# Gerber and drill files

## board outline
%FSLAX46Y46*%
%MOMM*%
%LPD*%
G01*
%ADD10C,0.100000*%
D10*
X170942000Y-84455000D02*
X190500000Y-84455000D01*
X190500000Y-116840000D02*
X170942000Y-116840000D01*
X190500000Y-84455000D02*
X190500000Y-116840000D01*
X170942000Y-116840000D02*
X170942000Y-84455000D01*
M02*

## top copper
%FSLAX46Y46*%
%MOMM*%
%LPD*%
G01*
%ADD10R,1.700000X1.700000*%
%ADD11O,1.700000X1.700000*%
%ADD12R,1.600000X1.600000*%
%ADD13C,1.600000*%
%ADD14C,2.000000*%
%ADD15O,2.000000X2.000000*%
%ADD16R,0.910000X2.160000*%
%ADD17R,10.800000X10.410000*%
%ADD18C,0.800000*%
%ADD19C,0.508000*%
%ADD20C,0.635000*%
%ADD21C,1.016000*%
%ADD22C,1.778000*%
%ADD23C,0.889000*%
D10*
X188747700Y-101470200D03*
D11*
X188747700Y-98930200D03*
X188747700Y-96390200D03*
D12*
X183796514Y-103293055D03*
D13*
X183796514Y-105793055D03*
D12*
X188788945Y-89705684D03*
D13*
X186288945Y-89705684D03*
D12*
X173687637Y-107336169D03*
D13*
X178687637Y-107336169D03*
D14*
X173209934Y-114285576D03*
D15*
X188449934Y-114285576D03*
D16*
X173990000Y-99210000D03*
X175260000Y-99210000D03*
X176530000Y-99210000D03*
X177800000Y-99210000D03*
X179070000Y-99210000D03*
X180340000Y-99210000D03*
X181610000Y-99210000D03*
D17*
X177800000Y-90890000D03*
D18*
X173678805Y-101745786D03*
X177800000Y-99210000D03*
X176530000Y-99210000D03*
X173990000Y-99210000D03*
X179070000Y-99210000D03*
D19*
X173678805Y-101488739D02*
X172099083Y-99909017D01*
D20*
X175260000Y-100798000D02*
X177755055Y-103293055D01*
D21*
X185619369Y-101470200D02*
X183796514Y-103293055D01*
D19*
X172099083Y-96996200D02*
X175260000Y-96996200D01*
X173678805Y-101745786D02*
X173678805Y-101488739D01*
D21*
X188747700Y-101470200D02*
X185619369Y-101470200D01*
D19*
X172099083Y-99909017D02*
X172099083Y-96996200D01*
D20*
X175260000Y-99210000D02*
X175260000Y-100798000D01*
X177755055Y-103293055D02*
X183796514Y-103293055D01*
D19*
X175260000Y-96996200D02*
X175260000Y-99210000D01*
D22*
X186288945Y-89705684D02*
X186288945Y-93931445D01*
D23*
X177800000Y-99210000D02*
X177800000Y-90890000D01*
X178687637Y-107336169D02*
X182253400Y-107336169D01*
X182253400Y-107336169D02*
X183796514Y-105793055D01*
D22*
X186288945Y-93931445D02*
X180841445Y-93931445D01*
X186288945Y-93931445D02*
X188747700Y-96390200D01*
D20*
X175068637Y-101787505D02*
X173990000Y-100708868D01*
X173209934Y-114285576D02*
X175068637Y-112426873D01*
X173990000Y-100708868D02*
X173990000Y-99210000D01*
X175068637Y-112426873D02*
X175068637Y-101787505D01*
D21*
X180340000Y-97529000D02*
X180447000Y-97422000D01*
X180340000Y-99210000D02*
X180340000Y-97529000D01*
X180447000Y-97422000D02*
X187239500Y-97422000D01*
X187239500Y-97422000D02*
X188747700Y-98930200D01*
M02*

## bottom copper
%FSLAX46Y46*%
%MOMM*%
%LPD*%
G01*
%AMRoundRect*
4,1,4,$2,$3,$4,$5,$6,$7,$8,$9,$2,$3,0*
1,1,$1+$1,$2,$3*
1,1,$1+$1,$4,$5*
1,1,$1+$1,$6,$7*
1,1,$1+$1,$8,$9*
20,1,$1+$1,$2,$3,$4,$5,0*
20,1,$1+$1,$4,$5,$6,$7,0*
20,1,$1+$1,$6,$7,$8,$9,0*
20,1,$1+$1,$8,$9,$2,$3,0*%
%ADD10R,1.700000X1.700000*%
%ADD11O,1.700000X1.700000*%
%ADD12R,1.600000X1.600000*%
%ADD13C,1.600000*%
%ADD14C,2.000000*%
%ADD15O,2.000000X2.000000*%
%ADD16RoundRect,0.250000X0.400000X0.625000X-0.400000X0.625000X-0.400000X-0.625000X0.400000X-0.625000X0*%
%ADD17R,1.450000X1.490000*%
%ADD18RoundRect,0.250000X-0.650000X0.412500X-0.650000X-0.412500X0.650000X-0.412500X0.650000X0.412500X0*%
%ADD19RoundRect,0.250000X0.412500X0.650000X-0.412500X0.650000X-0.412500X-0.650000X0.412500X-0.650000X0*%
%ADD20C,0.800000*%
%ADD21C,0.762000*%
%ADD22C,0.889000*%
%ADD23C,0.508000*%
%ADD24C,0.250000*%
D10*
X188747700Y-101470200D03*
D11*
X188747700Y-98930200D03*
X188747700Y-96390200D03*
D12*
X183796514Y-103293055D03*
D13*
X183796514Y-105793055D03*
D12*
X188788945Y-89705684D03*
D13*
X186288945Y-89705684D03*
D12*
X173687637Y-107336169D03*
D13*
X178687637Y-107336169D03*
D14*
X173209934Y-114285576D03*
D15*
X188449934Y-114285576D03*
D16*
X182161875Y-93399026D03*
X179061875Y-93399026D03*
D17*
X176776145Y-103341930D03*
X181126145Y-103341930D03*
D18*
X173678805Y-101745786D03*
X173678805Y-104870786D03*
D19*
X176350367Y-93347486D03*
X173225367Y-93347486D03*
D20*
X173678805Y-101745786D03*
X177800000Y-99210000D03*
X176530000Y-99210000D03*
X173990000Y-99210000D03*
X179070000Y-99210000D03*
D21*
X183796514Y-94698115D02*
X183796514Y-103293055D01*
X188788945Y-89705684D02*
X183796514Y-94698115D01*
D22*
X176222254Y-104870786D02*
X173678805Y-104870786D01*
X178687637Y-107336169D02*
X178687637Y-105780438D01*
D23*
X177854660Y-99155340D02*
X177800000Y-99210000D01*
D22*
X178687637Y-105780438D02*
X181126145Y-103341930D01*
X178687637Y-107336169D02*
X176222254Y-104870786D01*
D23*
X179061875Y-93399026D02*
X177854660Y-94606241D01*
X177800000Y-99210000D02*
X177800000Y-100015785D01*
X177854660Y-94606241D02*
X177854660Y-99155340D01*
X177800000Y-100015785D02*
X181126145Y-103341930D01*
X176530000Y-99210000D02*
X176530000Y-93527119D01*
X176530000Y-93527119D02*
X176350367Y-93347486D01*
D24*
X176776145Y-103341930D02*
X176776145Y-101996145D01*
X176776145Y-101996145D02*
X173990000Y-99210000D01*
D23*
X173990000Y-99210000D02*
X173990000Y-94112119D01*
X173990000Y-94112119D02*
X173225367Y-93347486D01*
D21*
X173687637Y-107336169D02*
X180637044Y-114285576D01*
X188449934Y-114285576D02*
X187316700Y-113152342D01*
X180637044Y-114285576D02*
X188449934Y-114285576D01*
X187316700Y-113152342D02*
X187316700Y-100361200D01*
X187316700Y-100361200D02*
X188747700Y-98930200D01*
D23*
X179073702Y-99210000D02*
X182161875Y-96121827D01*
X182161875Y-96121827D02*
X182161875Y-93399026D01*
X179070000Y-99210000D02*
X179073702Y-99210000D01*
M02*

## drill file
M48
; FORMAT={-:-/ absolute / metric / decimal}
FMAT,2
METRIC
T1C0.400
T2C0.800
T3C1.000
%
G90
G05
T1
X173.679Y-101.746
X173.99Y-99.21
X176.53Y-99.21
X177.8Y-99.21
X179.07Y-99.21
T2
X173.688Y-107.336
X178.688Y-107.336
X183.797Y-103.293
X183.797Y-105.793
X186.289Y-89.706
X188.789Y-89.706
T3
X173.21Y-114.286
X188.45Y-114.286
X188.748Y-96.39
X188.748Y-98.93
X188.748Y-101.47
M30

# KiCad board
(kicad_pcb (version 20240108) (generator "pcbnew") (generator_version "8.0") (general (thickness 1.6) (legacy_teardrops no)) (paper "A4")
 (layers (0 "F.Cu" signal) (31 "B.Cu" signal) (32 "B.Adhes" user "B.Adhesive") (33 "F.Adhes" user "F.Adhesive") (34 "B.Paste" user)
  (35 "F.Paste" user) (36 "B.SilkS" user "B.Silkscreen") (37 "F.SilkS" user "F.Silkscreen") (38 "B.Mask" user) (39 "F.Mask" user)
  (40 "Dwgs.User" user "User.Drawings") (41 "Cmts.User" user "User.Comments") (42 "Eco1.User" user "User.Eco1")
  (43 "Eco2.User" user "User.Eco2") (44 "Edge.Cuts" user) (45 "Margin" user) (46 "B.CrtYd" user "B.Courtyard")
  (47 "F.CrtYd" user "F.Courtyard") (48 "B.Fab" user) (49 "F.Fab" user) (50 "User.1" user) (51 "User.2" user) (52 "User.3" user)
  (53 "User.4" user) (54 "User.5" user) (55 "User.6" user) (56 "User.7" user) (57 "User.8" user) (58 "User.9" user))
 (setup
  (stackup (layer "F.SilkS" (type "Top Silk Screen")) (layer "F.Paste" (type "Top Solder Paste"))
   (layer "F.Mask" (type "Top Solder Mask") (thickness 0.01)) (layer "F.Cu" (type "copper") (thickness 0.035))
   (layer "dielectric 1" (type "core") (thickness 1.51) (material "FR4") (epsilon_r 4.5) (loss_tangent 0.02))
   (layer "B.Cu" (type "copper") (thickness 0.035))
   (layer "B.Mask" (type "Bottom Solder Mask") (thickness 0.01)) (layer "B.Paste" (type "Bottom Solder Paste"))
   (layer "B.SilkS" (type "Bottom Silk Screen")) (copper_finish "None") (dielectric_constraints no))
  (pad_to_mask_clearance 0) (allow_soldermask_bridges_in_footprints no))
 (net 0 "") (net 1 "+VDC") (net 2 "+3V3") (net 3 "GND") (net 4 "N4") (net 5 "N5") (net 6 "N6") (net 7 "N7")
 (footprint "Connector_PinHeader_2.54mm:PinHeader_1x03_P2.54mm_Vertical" (layer "F.Cu") (at 188.7477 101.4702 180)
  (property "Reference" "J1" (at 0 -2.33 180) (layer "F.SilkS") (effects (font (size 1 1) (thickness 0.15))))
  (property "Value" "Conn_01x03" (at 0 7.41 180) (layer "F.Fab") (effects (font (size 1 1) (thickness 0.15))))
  (pad "1" thru_hole rect (at 0 0 180) (size 1.7 1.7) (drill 1) (layers "*.Cu" "*.Mask") (remove_unused_layers no) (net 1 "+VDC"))
  (pad "2" thru_hole oval (at 0 2.54 180) (size 1.7 1.7) (drill 1) (layers "*.Cu" "*.Mask") (remove_unused_layers no) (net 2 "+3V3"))
  (pad "3" thru_hole oval (at 0 5.08 180) (size 1.7 1.7) (drill 1) (layers "*.Cu" "*.Mask") (remove_unused_layers no) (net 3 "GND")))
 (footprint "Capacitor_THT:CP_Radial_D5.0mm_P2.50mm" (layer "F.Cu") (at 183.796514 103.293055 -90)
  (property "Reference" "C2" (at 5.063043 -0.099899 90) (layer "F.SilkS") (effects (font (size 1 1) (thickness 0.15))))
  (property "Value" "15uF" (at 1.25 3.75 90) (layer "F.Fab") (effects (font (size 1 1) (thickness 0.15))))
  (pad "1" thru_hole rect (at 0 0 270) (size 1.6 1.6) (drill 0.8) (layers "*.Cu" "*.Mask") (remove_unused_layers no) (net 1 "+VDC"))
  (pad "2" thru_hole circle (at 2.5 0 270) (size 1.6 1.6) (drill 0.8) (layers "*.Cu" "*.Mask") (remove_unused_layers no) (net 3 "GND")))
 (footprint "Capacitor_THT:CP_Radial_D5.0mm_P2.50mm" (layer "F.Cu") (at 188.788945 89.705684 180)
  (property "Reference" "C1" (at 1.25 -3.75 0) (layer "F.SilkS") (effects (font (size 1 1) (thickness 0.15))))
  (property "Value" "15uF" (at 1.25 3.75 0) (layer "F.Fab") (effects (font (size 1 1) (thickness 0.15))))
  (pad "1" thru_hole rect (at 0 0 180) (size 1.6 1.6) (drill 0.8) (layers "*.Cu" "*.Mask") (remove_unused_layers no) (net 1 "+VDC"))
  (pad "2" thru_hole circle (at 2.5 0 180) (size 1.6 1.6) (drill 0.8) (layers "*.Cu" "*.Mask") (remove_unused_layers no) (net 3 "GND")))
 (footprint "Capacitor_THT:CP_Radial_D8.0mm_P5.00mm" (layer "F.Cu") (at 173.687637 107.336169)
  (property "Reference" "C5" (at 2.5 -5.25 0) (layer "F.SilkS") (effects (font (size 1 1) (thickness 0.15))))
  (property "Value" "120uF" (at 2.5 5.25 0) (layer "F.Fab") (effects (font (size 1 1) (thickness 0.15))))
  (pad "1" thru_hole rect (at 0 0) (size 1.6 1.6) (drill 0.8) (layers "*.Cu" "*.Mask") (remove_unused_layers no) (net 2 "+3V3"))
  (pad "2" thru_hole circle (at 5 0) (size 1.6 1.6) (drill 0.8) (layers "*.Cu" "*.Mask") (remove_unused_layers no) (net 3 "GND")))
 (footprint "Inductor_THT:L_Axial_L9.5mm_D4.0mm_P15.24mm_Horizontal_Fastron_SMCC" (layer "F.Cu") (at 173.209934 114.285576)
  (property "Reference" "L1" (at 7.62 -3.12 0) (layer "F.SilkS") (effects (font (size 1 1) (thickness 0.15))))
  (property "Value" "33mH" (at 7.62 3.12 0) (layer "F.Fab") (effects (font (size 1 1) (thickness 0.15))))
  (pad "1" thru_hole circle (at 0 0) (size 2 2) (drill 1) (layers "*.Cu" "*.Mask") (remove_unused_layers no) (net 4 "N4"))
  (pad "2" thru_hole oval (at 15.24 0) (size 2 2) (drill 1) (layers "*.Cu" "*.Mask") (remove_unused_layers no) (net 2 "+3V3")))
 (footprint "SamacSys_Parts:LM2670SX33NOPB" (layer "F.Cu") (at 177.8 91.44 -90)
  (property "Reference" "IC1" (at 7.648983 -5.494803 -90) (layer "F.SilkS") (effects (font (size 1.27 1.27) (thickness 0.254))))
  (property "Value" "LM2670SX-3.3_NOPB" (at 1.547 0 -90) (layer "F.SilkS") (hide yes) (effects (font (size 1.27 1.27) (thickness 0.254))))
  (pad "1" smd rect (at 7.77 3.81) (size 0.91 2.16) (layers "F.Cu" "F.Paste" "F.Mask") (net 4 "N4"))
  (pad "2" smd rect (at 7.77 2.54) (size 0.91 2.16) (layers "F.Cu" "F.Paste" "F.Mask") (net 1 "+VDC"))
  (pad "3" smd rect (at 7.77 1.27) (size 0.91 2.16) (layers "F.Cu" "F.Paste" "F.Mask") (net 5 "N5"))
  (pad "4" smd rect (at 7.77 0) (size 0.91 2.16) (layers "F.Cu" "F.Paste" "F.Mask") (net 3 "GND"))
  (pad "5" smd rect (at 7.77 -1.27) (size 0.91 2.16) (layers "F.Cu" "F.Paste" "F.Mask") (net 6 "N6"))
  (pad "6" smd rect (at 7.77 -2.54) (size 0.91 2.16) (layers "F.Cu" "F.Paste" "F.Mask") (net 2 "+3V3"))
  (pad "7" smd rect (at 7.77 -3.81) (size 0.91 2.16) (layers "F.Cu" "F.Paste" "F.Mask") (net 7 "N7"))
  (pad "8" smd rect (at -0.55 0 270) (size 10.41 10.8) (layers "F.Cu" "F.Paste" "F.Mask") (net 3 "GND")))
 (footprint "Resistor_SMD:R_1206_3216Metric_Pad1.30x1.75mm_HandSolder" (layer "B.Cu") (at 180.611875 93.399026 180)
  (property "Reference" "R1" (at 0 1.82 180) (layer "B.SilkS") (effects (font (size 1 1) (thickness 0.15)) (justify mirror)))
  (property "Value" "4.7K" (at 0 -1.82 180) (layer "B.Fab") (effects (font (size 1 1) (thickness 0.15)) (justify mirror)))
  (pad "1" smd roundrect (at -1.55 0 180) (size 1.3 1.75) (layers "B.Cu" "B.Paste" "B.Mask") (roundrect_rratio 0.192308) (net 6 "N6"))
  (pad "2" smd roundrect (at 1.55 0 180) (size 1.3 1.75) (layers "B.Cu" "B.Paste" "B.Mask") (roundrect_rratio 0.192308) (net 3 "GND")))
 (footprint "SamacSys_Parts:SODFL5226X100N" (layer "B.Cu") (at 178.951145 103.34193)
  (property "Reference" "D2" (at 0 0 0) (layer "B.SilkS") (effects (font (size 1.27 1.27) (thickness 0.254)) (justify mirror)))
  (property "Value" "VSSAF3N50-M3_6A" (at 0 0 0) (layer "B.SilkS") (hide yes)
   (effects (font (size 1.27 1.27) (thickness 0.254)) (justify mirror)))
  (pad "1" smd rect (at -2.175 0) (size 1.45 1.49) (layers "B.Cu" "B.Paste" "B.Mask") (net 4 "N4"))
  (pad "2" smd rect (at 2.175 0) (size 1.45 1.49) (layers "B.Cu" "B.Paste" "B.Mask") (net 3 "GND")))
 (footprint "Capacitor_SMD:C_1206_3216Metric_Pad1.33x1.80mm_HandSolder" (layer "B.Cu") (at 173.678805 103.308286 -90)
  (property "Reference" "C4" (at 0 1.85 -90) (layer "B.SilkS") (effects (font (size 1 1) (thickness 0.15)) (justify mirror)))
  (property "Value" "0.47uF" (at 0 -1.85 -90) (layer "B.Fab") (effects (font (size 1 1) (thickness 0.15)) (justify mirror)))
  (pad "1" smd roundrect (at -1.5625 0 270) (size 1.325 1.8) (layers "B.Cu" "B.Paste" "B.Mask") (roundrect_rratio 0.188679) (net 1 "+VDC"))
  (pad "2" smd roundrect (at 1.5625 0 270) (size 1.325 1.8) (layers "B.Cu" "B.Paste" "B.Mask") (roundrect_rratio 0.188679) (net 3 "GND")))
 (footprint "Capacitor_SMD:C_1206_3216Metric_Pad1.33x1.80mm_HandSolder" (layer "B.Cu") (at 174.787867 93.347486 180)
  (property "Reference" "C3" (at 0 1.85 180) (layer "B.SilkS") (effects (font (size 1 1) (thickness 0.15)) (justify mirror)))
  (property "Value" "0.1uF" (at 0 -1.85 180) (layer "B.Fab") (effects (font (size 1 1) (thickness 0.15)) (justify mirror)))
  (pad "1" smd roundrect (at -1.5625 0 180) (size 1.325 1.8) (layers "B.Cu" "B.Paste" "B.Mask") (roundrect_rratio 0.188679) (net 5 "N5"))
  (pad "2" smd roundrect (at 1.5625 0 180) (size 1.325 1.8) (layers "B.Cu" "B.Paste" "B.Mask") (roundrect_rratio 0.188679) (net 4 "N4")))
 (gr_line (start 170.942 84.455) (end 190.5 84.455) (stroke (width 0.1) (type solid)) (layer "Edge.Cuts"))
 (gr_line (start 190.5 116.84) (end 170.942 116.84) (stroke (width 0.1) (type default)) (layer "Edge.Cuts"))
 (gr_line (start 190.5 84.455) (end 190.5 116.84) (stroke (width 0.1) (type default)) (layer "Edge.Cuts"))
 (gr_line (start 170.942 116.84) (end 170.942 84.455) (stroke (width 0.1) (type solid)) (layer "Edge.Cuts"))
 (segment (start 173.678805 101.488739) (end 172.099083 99.909017) (width 0.508) (layer "F.Cu") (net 1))
 (segment (start 175.26 100.798) (end 177.755055 103.293055) (width 0.635) (layer "F.Cu") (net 1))
 (segment (start 185.619369 101.4702) (end 183.796514 103.293055) (width 1.016) (layer "F.Cu") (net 1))
 (segment (start 172.099083 96.9962) (end 175.26 96.9962) (width 0.508) (layer "F.Cu") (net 1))
 (segment (start 173.678805 101.745786) (end 173.678805 101.488739) (width 0.508) (layer "F.Cu") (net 1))
 (segment (start 188.7477 101.4702) (end 185.619369 101.4702) (width 1.016) (layer "F.Cu") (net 1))
 (segment (start 172.099083 99.909017) (end 172.099083 96.9962) (width 0.508) (layer "F.Cu") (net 1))
 (segment (start 175.26 99.21) (end 175.26 100.798) (width 0.635) (layer "F.Cu") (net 1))
 (segment (start 177.755055 103.293055) (end 183.796514 103.293055) (width 0.635) (layer "F.Cu") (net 1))
 (segment (start 175.26 96.9962) (end 175.26 99.21) (width 0.508) (layer "F.Cu") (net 1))
 (via (at 173.678805 101.745786) (size 0.8) (drill 0.4) (layers "F.Cu" "B.Cu") (free yes) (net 1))
 (segment (start 183.796514 94.698115) (end 183.796514 103.293055) (width 0.762) (layer "B.Cu") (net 1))
 (segment (start 188.788945 89.705684) (end 183.796514 94.698115) (width 0.762) (layer "B.Cu") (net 1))
 (segment (start 186.288945 89.705684) (end 186.288945 93.931445) (width 1.778) (layer "F.Cu") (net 3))
 (segment (start 177.8 99.21) (end 177.8 90.89) (width 0.889) (layer "F.Cu") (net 3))
 (segment (start 178.687637 107.336169) (end 182.2534 107.336169) (width 0.889) (layer "F.Cu") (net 3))
 (segment (start 182.2534 107.336169) (end 183.796514 105.793055) (width 0.889) (layer "F.Cu") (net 3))
 (segment (start 186.288945 93.931445) (end 180.841445 93.931445) (width 1.778) (layer "F.Cu") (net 3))
 (segment (start 186.288945 93.931445) (end 188.7477 96.3902) (width 1.778) (layer "F.Cu") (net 3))
 (via (at 177.8 99.21) (size 0.8) (drill 0.4) (layers "F.Cu" "B.Cu") (free yes) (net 3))
 (segment (start 176.222254 104.870786) (end 173.678805 104.870786) (width 0.889) (layer "B.Cu") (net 3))
 (segment (start 178.687637 107.336169) (end 178.687637 105.780438) (width 0.889) (layer "B.Cu") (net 3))
 (segment (start 177.85466 99.15534) (end 177.8 99.21) (width 0.508) (layer "B.Cu") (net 3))
 (segment (start 178.687637 105.780438) (end 181.126145 103.34193) (width 0.889) (layer "B.Cu") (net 3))
 (segment (start 178.687637 107.336169) (end 176.222254 104.870786) (width 0.889) (layer "B.Cu") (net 3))
 (segment (start 179.061875 93.399026) (end 177.85466 94.606241) (width 0.508) (layer "B.Cu") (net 3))
 (segment (start 177.8 99.21) (end 177.8 100.015785) (width 0.508) (layer "B.Cu") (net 3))
 (segment (start 177.85466 94.606241) (end 177.85466 99.15534) (width 0.508) (layer "B.Cu") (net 3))
 (segment (start 177.8 100.015785) (end 181.126145 103.34193) (width 0.508) (layer "B.Cu") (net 3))
 (via (at 176.53 99.21) (size 0.8) (drill 0.4) (layers "F.Cu" "B.Cu") (free yes) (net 5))
 (segment (start 176.53 99.21) (end 176.53 93.527119) (width 0.508) (layer "B.Cu") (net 5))
 (segment (start 176.53 93.527119) (end 176.350367 93.347486) (width 0.508) (layer "B.Cu") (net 5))
 (segment (start 175.068637 101.787505) (end 173.99 100.708868) (width 0.635) (layer "F.Cu") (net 4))
 (segment (start 173.209934 114.285576) (end 175.068637 112.426873) (width 0.635) (layer "F.Cu") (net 4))
 (segment (start 173.99 100.708868) (end 173.99 99.21) (width 0.635) (layer "F.Cu") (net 4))
 (segment (start 175.068637 112.426873) (end 175.068637 101.787505) (width 0.635) (layer "F.Cu") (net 4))
 (via (at 173.99 99.21) (size 0.8) (drill 0.4) (layers "F.Cu" "B.Cu") (free yes) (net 4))
 (segment (start 176.776145 103.34193) (end 176.776145 101.996145) (width 0.25) (layer "B.Cu") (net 4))
 (segment (start 176.776145 101.996145) (end 173.99 99.21) (width 0.25) (layer "B.Cu") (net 4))
 (segment (start 173.99 99.21) (end 173.99 94.112119) (width 0.508) (layer "B.Cu") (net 4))
 (segment (start 173.99 94.112119) (end 173.225367 93.347486) (width 0.508) (layer "B.Cu") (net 4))
 (segment (start 180.34 97.529) (end 180.447 97.422) (width 1.016) (layer "F.Cu") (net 2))
 (segment (start 180.34 99.21) (end 180.34 97.529) (width 1.016) (layer "F.Cu") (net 2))
 (segment (start 180.447 97.422) (end 187.2395 97.422) (width 1.016) (layer "F.Cu") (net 2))
 (segment (start 187.2395 97.422) (end 188.7477 98.9302) (width 1.016) (layer "F.Cu") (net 2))
 (segment (start 173.687637 107.336169) (end 180.637044 114.285576) (width 0.762) (layer "B.Cu") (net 2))
 (segment (start 188.449934 114.285576) (end 187.3167 113.152342) (width 0.762) (layer "B.Cu") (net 2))
 (segment (start 180.637044 114.285576) (end 188.449934 114.285576) (width 0.762) (layer "B.Cu") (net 2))
 (segment (start 187.3167 113.152342) (end 187.3167 100.3612) (width 0.762) (layer "B.Cu") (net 2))
 (segment (start 187.3167 100.3612) (end 188.7477 98.9302) (width 0.762) (layer "B.Cu") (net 2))
 (via (at 179.07 99.21) (size 0.8) (drill 0.4) (layers "F.Cu" "B.Cu") (free yes) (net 6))
 (segment (start 179.073702 99.21) (end 182.161875 96.121827) (width 0.508) (layer "B.Cu") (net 6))
 (segment (start 182.161875 96.121827) (end 182.161875 93.399026) (width 0.508) (layer "B.Cu") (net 6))
 (segment (start 179.07 99.21) (end 179.073702 99.21) (width 0.508) (layer "B.Cu") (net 6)))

